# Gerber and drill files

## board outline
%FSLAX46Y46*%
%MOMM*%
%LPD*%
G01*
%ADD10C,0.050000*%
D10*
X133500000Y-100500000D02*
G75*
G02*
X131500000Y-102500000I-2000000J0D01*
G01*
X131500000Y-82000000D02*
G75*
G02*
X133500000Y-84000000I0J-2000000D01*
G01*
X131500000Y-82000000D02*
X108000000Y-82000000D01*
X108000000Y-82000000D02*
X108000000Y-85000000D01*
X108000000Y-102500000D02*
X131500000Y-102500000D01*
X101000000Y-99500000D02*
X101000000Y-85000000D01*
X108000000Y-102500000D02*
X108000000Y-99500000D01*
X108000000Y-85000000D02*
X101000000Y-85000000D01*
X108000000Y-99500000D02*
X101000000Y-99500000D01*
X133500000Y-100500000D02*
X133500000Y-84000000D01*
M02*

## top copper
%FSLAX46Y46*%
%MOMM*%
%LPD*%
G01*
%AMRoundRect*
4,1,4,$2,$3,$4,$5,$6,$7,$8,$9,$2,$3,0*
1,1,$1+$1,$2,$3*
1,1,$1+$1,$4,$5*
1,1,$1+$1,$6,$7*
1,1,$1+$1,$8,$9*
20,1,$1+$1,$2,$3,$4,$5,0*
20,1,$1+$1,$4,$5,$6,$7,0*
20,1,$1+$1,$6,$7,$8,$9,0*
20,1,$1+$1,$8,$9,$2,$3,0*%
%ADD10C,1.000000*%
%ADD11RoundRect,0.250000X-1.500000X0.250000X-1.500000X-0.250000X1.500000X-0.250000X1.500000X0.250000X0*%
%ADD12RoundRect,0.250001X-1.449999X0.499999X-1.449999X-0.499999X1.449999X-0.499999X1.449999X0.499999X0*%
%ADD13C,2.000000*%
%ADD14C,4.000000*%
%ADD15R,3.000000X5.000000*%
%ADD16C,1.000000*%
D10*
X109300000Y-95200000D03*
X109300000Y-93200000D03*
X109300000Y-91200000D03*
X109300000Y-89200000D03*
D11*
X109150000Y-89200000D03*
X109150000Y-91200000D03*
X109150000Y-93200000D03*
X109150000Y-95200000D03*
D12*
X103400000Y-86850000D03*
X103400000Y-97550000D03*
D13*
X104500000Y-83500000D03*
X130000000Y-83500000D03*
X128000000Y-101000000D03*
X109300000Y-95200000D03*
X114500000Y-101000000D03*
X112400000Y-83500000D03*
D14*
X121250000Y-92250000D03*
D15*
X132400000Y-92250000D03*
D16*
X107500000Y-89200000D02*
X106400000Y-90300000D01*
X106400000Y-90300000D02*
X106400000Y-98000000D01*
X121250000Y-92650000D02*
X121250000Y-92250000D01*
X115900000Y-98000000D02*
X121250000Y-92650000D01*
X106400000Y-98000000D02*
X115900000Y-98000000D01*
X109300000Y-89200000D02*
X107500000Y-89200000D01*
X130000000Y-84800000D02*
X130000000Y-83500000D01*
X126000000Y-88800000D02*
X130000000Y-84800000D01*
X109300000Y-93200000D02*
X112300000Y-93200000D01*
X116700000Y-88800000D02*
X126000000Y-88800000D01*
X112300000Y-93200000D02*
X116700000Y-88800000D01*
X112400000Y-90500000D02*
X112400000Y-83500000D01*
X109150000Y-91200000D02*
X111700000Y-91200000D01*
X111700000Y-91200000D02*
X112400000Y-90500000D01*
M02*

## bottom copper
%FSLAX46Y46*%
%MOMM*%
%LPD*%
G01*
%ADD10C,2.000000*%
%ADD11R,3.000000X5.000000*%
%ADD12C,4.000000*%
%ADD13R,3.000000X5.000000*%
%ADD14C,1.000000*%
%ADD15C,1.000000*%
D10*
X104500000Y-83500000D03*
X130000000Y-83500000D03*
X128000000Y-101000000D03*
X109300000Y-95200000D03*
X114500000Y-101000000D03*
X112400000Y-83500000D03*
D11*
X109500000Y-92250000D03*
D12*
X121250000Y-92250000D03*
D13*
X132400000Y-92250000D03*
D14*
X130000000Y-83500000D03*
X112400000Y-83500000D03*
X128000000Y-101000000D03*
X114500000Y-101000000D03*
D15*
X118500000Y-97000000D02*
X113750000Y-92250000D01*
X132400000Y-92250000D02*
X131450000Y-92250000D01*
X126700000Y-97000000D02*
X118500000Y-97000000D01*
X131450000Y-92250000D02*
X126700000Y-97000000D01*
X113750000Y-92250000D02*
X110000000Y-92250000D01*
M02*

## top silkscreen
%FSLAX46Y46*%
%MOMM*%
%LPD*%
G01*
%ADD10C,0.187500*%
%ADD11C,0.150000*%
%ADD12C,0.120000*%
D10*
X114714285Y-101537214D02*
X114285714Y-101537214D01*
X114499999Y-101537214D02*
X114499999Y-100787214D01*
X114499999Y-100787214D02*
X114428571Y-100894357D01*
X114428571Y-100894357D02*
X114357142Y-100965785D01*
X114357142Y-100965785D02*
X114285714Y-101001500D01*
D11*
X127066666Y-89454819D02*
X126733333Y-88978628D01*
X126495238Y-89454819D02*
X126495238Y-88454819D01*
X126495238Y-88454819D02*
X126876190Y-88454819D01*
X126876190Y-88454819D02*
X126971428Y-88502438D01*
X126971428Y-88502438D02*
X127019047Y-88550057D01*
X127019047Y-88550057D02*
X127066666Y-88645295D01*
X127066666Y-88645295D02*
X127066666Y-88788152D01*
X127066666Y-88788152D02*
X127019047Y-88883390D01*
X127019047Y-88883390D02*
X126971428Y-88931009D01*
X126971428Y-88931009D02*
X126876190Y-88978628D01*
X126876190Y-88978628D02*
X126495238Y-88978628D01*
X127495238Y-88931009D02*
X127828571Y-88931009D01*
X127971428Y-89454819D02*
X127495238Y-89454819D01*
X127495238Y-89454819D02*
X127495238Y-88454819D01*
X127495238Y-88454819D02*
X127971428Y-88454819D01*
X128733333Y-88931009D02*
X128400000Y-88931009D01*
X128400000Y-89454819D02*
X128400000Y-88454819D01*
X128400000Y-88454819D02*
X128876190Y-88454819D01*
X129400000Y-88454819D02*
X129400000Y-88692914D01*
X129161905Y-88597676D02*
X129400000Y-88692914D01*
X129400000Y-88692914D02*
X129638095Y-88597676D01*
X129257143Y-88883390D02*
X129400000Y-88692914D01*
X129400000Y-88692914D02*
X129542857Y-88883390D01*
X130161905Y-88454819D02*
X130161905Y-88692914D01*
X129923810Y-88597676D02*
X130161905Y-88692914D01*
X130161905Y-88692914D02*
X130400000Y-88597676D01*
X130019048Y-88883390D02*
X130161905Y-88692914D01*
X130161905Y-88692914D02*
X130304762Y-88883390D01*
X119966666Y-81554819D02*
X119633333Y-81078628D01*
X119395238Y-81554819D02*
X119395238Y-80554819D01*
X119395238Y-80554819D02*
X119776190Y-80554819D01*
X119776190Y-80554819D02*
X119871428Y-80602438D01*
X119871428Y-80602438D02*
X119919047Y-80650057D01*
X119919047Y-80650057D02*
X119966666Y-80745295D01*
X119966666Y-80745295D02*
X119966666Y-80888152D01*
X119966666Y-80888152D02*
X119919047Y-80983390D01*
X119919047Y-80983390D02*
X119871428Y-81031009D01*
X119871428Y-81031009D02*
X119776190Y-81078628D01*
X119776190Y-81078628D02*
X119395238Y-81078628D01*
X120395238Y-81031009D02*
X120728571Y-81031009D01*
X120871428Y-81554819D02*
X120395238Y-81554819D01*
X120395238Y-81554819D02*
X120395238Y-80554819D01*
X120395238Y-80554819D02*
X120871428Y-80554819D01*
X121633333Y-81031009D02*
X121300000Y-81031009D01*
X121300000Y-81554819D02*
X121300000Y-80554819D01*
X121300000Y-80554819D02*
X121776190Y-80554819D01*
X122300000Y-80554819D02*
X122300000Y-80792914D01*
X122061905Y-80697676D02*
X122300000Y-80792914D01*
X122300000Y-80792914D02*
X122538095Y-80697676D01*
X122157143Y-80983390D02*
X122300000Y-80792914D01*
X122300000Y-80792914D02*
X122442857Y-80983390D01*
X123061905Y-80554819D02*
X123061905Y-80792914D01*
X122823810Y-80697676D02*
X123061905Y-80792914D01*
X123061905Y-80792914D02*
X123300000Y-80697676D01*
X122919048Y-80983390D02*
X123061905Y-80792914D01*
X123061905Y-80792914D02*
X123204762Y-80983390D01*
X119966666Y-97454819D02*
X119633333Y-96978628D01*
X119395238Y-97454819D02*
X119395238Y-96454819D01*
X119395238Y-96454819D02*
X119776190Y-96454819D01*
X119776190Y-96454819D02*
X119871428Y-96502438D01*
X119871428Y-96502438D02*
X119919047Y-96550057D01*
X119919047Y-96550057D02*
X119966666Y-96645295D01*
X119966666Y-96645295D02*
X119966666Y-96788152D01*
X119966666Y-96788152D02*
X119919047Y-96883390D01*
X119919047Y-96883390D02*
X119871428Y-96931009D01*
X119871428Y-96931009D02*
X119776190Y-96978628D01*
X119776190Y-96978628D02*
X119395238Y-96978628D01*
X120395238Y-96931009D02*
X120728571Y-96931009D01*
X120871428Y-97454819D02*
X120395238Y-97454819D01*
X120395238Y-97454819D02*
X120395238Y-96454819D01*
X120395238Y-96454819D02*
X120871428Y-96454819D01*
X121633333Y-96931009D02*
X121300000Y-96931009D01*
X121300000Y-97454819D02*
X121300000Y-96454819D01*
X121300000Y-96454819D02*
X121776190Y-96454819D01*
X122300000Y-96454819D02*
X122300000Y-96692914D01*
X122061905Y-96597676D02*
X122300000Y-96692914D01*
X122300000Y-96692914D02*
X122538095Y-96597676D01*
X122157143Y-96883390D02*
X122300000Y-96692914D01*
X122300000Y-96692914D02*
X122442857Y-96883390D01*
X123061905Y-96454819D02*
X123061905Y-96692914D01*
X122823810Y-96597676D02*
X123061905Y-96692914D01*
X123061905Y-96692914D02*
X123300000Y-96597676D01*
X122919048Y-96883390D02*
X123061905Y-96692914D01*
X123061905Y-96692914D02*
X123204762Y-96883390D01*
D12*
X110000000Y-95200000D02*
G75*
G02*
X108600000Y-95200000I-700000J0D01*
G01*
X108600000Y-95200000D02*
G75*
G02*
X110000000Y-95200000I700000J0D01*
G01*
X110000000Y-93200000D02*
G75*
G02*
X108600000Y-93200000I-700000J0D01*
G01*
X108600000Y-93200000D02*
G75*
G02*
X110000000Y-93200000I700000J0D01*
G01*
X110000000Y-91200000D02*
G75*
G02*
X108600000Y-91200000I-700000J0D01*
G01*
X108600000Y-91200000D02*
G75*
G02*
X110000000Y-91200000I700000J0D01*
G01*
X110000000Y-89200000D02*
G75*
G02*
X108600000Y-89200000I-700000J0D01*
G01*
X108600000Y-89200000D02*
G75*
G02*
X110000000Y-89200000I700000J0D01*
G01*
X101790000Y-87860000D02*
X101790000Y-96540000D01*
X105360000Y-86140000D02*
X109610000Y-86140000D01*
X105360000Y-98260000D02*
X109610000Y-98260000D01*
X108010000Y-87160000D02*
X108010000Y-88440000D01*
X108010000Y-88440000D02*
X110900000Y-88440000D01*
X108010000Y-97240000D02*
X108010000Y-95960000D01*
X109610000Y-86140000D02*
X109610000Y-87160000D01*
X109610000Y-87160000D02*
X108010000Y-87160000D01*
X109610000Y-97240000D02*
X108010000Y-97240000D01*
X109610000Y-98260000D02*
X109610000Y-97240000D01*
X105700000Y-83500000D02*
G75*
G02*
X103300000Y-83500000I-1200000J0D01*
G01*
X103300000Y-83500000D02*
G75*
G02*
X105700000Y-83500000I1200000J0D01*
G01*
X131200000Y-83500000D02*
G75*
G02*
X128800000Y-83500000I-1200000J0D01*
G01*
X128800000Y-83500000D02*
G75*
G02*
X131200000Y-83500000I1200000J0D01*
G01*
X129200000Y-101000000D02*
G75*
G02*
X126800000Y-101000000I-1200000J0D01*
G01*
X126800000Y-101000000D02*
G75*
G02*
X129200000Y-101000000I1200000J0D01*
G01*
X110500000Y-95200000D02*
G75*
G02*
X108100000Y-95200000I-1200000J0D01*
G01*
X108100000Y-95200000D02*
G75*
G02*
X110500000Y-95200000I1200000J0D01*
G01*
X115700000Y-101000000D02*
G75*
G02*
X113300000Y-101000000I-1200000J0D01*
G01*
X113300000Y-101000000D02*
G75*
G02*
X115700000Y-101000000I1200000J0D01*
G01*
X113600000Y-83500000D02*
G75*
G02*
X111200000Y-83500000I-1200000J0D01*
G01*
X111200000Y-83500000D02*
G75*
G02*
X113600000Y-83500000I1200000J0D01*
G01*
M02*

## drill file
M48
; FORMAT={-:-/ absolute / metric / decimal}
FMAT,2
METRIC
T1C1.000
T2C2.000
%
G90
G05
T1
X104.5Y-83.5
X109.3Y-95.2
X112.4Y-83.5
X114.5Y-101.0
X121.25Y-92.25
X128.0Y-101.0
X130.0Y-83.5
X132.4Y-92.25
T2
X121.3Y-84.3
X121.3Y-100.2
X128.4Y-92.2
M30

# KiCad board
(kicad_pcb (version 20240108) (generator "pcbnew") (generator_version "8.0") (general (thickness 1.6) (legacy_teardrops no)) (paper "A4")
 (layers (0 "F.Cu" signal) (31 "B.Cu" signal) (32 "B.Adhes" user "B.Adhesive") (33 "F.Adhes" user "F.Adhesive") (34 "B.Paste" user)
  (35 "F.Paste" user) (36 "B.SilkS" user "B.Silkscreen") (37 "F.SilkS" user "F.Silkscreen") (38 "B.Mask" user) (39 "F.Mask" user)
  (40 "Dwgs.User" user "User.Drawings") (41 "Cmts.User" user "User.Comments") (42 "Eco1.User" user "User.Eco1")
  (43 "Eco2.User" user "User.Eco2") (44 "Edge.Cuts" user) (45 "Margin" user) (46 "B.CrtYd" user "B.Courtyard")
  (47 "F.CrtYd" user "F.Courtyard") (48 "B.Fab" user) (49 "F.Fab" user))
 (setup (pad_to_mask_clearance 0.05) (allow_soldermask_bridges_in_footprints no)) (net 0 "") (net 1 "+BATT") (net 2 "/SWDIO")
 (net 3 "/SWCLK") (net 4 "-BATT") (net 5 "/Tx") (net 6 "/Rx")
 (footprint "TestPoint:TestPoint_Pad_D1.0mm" (layer "F.Cu") (at 109.3 95.2)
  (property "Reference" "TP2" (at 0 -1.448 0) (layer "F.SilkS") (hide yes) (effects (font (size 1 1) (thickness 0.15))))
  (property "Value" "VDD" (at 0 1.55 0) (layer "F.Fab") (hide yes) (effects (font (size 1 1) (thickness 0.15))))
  (fp_circle (center 0 0) (end 0 0.7) (stroke (width 0.12) (type solid)) (fill none) (layer "F.SilkS"))
  (pad "1" smd circle (at 0 0) (size 1 1) (layers "F.Cu" "F.Mask") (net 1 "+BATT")))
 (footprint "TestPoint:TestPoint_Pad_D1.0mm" (layer "F.Cu") (at 109.3 93.2)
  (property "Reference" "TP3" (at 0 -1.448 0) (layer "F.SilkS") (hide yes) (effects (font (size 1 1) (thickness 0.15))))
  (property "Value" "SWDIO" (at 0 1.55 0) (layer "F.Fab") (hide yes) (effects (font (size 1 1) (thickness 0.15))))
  (fp_circle (center 0 0) (end 0 0.7) (stroke (width 0.12) (type solid)) (fill none) (layer "F.SilkS"))
  (pad "1" smd circle (at 0 0) (size 1 1) (layers "F.Cu" "F.Mask") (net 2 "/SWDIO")))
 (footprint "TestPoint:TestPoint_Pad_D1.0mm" (layer "F.Cu") (at 109.3 91.2)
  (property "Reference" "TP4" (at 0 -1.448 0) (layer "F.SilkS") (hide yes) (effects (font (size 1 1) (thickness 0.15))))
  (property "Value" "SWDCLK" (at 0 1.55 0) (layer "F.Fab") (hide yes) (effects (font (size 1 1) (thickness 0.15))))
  (fp_circle (center 0 0) (end 0 0.7) (stroke (width 0.12) (type solid)) (fill none) (layer "F.SilkS"))
  (pad "1" smd circle (at 0 0) (size 1 1) (layers "F.Cu" "F.Mask") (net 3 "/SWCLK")))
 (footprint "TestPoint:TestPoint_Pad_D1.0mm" (layer "F.Cu") (at 109.3 89.2)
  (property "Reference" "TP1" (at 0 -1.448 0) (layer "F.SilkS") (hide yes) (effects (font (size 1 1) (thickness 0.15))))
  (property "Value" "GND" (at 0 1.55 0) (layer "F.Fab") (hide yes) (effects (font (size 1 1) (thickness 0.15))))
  (fp_circle (center 0 0) (end 0 0.7) (stroke (width 0.12) (type solid)) (fill none) (layer "F.SilkS"))
  (pad "1" smd circle (at 0 0) (size 1 1) (layers "F.Cu" "F.Mask") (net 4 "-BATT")))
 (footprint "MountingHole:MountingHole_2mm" (layer "F.Cu") (at 128.4 92.2)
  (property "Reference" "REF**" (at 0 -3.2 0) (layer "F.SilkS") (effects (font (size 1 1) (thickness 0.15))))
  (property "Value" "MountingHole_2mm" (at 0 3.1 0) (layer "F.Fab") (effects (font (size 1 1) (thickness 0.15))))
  (pad "" np_thru_hole circle (at 0 0) (size 2 2) (drill 2) (layers "*.Cu" "*.Mask")))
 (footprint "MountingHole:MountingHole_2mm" (layer "F.Cu") (at 121.3 84.3)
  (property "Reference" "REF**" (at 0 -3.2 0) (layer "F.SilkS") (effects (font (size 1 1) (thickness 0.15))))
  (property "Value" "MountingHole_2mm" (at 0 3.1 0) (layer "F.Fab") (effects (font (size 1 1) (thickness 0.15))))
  (pad "" np_thru_hole circle (at 0 0) (size 2 2) (drill 2) (layers "*.Cu" "*.Mask")))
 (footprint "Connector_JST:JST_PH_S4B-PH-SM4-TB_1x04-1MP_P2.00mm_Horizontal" (layer "F.Cu") (at 106.3 92.2 -90)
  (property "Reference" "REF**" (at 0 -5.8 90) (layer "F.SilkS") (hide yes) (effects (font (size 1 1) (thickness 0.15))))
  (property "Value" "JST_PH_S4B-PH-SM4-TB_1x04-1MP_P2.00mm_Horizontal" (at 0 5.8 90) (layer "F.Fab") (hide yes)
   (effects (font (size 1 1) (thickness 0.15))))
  (fp_line (start -4.34 4.51) (end 4.34 4.51) (stroke (width 0.12) (type solid)) (layer "F.SilkS"))
  (fp_line (start -6.06 0.94) (end -6.06 -3.31) (stroke (width 0.12) (type solid)) (layer "F.SilkS"))
  (fp_line (start 6.06 0.94) (end 6.06 -3.31) (stroke (width 0.12) (type solid)) (layer "F.SilkS"))
  (fp_line (start -5.04 -1.71) (end -3.76 -1.71) (stroke (width 0.12) (type solid)) (layer "F.SilkS"))
  (fp_line (start -3.76 -1.71) (end -3.76 -4.6) (stroke (width 0.12) (type solid)) (layer "F.SilkS"))
  (fp_line (start 5.04 -1.71) (end 3.76 -1.71) (stroke (width 0.12) (type solid)) (layer "F.SilkS"))
  (fp_line (start -6.06 -3.31) (end -5.04 -3.31) (stroke (width 0.12) (type solid)) (layer "F.SilkS"))
  (fp_line (start -5.04 -3.31) (end -5.04 -1.71) (stroke (width 0.12) (type solid)) (layer "F.SilkS"))
  (fp_line (start 5.04 -3.31) (end 5.04 -1.71) (stroke (width 0.12) (type solid)) (layer "F.SilkS"))
  (fp_line (start 6.06 -3.31) (end 5.04 -3.31) (stroke (width 0.12) (type solid)) (layer "F.SilkS"))
  (pad "1" smd roundrect (at -3 -2.85 270) (size 1 3.5) (layers "F.Cu" "F.Paste" "F.Mask") (roundrect_rratio 0.25) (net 4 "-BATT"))
  (pad "2" smd roundrect (at -1 -2.85 270) (size 1 3.5) (layers "F.Cu" "F.Paste" "F.Mask") (roundrect_rratio 0.25) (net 3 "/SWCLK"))
  (pad "3" smd roundrect (at 1 -2.85 270) (size 1 3.5) (layers "F.Cu" "F.Paste" "F.Mask") (roundrect_rratio 0.25) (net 2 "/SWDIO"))
  (pad "4" smd roundrect (at 3 -2.85 270) (size 1 3.5) (layers "F.Cu" "F.Paste" "F.Mask") (roundrect_rratio 0.25) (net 1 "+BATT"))
  (pad "MP" smd roundrect (at -5.35 2.9 270) (size 1.5 3.4) (layers "F.Cu" "F.Paste" "F.Mask") (roundrect_rratio 0.166667))
  (pad "MP" smd roundrect (at 5.35 2.9 270) (size 1.5 3.4) (layers "F.Cu" "F.Paste" "F.Mask") (roundrect_rratio 0.166667)))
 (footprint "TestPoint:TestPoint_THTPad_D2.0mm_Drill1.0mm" (layer "F.Cu") (at 104.5 83.5)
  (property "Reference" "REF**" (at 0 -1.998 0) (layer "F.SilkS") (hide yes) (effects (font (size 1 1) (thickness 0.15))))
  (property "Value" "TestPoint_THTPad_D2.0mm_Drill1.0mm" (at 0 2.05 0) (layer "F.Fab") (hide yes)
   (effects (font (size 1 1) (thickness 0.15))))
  (fp_circle (center 0 0) (end 0 1.2) (stroke (width 0.12) (type solid)) (fill none) (layer "F.SilkS"))
  (pad "1" thru_hole circle (at 0 0) (size 2 2) (drill 1) (layers "*.Cu" "*.Mask") (remove_unused_layers no)))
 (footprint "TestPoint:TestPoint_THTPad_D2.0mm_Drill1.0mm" (layer "F.Cu") (at 130 83.5)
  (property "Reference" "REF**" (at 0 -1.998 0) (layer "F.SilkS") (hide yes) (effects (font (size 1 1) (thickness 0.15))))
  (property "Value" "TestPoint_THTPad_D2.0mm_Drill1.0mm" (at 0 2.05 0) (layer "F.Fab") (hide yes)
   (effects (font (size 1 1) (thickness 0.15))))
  (fp_circle (center 0 0) (end 0 1.2) (stroke (width 0.12) (type solid)) (fill none) (layer "F.SilkS"))
  (pad "1" thru_hole circle (at 0 0) (size 2 2) (drill 1) (layers "*.Cu" "*.Mask") (remove_unused_layers no) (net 2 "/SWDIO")))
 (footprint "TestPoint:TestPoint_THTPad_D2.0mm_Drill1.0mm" (layer "F.Cu") (at 128 101)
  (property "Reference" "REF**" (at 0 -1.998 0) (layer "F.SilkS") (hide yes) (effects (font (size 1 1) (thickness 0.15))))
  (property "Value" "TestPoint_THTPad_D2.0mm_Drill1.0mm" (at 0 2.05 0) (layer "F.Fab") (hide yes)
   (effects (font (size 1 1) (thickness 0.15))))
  (fp_circle (center 0 0) (end 0 1.2) (stroke (width 0.12) (type solid)) (fill none) (layer "F.SilkS"))
  (pad "1" thru_hole circle (at 0 0) (size 2 2) (drill 1) (layers "*.Cu" "*.Mask") (remove_unused_layers no) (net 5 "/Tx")))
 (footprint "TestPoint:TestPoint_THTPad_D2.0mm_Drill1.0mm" (layer "F.Cu") (at 109.3 95.2)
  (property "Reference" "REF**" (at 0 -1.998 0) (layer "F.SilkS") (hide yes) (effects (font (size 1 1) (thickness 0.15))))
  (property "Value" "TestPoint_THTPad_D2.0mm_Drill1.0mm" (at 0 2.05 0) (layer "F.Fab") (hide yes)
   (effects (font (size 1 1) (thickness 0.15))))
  (fp_circle (center 0 0) (end 0 1.2) (stroke (width 0.12) (type solid)) (fill none) (layer "F.SilkS"))
  (pad "1" thru_hole circle (at 0 0) (size 2 2) (drill 1) (layers "*.Cu" "*.Mask") (remove_unused_layers no) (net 1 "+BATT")))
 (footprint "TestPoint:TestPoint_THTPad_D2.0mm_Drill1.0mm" (layer "F.Cu") (at 114.5 101)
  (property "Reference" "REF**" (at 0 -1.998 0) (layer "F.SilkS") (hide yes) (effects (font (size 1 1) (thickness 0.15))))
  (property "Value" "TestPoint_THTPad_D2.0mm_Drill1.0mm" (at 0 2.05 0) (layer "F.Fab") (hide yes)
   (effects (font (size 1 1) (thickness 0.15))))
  (fp_circle (center 0 0) (end 0 1.2) (stroke (width 0.12) (type solid)) (fill none) (layer "F.SilkS"))
  (pad "1" thru_hole circle (at 0 0) (size 2 2) (drill 1) (layers "*.Cu" "*.Mask") (remove_unused_layers no) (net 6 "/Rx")))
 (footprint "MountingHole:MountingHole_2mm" (layer "F.Cu") (at 121.3 100.2)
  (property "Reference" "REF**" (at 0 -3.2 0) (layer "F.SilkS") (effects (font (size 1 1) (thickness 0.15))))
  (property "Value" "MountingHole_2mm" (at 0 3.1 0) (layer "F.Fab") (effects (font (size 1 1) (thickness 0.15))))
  (pad "" np_thru_hole circle (at 0 0) (size 2 2) (drill 2) (layers "*.Cu" "*.Mask")))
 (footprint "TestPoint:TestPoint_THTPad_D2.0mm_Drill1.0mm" (layer "F.Cu") (at 112.4 83.5)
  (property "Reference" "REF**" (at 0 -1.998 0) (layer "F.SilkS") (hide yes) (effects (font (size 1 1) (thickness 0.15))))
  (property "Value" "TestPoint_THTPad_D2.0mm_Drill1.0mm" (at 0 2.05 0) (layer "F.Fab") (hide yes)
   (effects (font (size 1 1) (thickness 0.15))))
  (fp_circle (center 0 0) (end 0 1.2) (stroke (width 0.12) (type solid)) (fill none) (layer "F.SilkS"))
  (pad "1" thru_hole circle (at 0 0) (size 2 2) (drill 1) (layers "*.Cu" "*.Mask") (remove_unused_layers no) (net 3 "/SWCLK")))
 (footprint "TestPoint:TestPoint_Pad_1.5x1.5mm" (layer "B.Cu") (at 110 92.25)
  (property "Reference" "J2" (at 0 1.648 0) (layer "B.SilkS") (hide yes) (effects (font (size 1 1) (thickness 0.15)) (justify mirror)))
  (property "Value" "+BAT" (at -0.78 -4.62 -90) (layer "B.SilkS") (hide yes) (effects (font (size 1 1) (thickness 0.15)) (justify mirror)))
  (pad "1" smd rect (at 0 0) (size 3 5) (drill (offset -0.5 0)) (layers "B.Cu" "B.Mask") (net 1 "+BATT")))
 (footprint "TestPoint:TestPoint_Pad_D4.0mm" (layer "B.Cu") (at 121.25 92.25)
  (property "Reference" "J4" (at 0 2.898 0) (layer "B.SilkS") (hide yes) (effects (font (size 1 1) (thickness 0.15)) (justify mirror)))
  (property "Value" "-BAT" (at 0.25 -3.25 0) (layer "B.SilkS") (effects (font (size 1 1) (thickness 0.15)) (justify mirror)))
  (pad "1" thru_hole circle (at 0 0) (size 4 4) (drill 1) (layers "*.Cu" "*.Mask") (remove_unused_layers no) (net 4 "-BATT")))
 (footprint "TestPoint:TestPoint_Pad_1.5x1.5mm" (layer "B.Cu") (at 132.4 92.25)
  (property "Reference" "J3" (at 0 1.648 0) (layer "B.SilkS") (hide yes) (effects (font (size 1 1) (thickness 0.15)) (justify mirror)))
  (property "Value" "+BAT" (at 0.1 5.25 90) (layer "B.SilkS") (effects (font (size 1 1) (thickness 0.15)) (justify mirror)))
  (pad "1" thru_hole rect (at 0 0) (size 3 5) (drill 1) (layers "*.Cu" "*.Mask") (remove_unused_layers no) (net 1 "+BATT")))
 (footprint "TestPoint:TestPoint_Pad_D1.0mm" (layer "B.Cu") (at 130 83.5)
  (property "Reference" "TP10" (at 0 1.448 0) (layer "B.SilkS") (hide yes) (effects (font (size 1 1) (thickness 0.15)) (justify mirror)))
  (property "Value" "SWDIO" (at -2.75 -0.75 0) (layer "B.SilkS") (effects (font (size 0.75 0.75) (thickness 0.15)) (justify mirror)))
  (pad "1" smd circle (at 0 0) (size 1 1) (layers "B.Cu" "B.Mask") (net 2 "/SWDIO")))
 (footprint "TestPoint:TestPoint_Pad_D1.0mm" (layer "B.Cu") (at 112.4 83.5)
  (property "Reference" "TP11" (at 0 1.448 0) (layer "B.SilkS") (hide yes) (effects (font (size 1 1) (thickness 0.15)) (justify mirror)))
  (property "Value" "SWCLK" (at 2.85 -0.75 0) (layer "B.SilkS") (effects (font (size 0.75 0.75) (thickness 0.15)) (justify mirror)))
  (pad "1" smd circle (at 0 0) (size 1 1) (layers "B.Cu" "B.Mask") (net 3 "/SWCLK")))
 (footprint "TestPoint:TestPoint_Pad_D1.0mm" (layer "B.Cu") (at 128 101 180)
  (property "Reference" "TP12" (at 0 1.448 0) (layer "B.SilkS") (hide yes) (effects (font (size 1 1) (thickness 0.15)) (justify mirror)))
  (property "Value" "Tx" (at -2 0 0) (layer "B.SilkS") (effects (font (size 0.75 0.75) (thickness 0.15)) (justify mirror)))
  (pad "1" smd circle (at 0 0 180) (size 1 1) (layers "B.Cu" "B.Mask") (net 5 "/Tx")))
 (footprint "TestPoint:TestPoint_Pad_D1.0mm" (layer "B.Cu") (at 114.5 101 180)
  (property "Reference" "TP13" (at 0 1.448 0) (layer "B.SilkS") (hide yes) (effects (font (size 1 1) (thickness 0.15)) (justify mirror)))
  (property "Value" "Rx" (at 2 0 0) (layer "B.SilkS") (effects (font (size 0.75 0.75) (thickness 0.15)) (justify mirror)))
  (pad "1" smd circle (at 0 0 180) (size 1 1) (layers "B.Cu" "B.Mask") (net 6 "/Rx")))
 (gr_arc (start 133.5 100.5) (mid 132.914214 101.914214) (end 131.5 102.5) (stroke (width 0.05) (type solid)) (layer "Edge.Cuts"))
 (gr_arc (start 131.5 82) (mid 132.914214 82.585786) (end 133.5 84) (stroke (width 0.05) (type solid)) (layer "Edge.Cuts"))
 (gr_line (start 131.5 82) (end 108 82) (stroke (width 0.05) (type solid)) (layer "Edge.Cuts"))
 (gr_line (start 108 82) (end 108 85) (stroke (width 0.05) (type default)) (layer "Edge.Cuts"))
 (gr_line (start 108 102.5) (end 131.5 102.5) (stroke (width 0.05) (type solid)) (layer "Edge.Cuts"))
 (gr_line (start 101 99.5) (end 101 85) (stroke (width 0.05) (type default)) (layer "Edge.Cuts"))
 (gr_line (start 108 102.5) (end 108 99.5) (stroke (width 0.05) (type default)) (layer "Edge.Cuts"))
 (gr_line (start 108 85) (end 101 85) (stroke (width 0.05) (type default)) (layer "Edge.Cuts"))
 (gr_line (start 108 99.5) (end 101 99.5) (stroke (width 0.05) (type default)) (layer "Edge.Cuts"))
 (gr_line (start 133.5 100.5) (end 133.5 84) (stroke (width 0.05) (type solid)) (layer "Edge.Cuts"))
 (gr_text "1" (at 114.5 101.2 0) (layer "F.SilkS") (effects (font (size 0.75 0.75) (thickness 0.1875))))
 (segment (start 118.5 97) (end 113.75 92.25) (width 1) (layer "B.Cu") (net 1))
 (segment (start 132.4 92.25) (end 131.45 92.25) (width 1) (layer "B.Cu") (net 1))
 (segment (start 126.7 97) (end 118.5 97) (width 1) (layer "B.Cu") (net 1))
 (segment (start 131.45 92.25) (end 126.7 97) (width 1) (layer "B.Cu") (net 1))
 (segment (start 113.75 92.25) (end 110 92.25) (width 1) (layer "B.Cu") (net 1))
 (segment (start 107.5 89.2) (end 106.4 90.3) (width 1) (layer "F.Cu") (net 4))
 (segment (start 106.4 90.3) (end 106.4 98) (width 1) (layer "F.Cu") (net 4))
 (segment (start 121.25 92.65) (end 121.25 92.25) (width 1) (layer "F.Cu") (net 4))
 (segment (start 115.9 98) (end 121.25 92.65) (width 1) (layer "F.Cu") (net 4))
 (segment (start 106.4 98) (end 115.9 98) (width 1) (layer "F.Cu") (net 4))
 (segment (start 109.3 89.2) (end 107.5 89.2) (width 1) (layer "F.Cu") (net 4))
 (segment (start 130 84.8) (end 130 83.5) (width 1) (layer "F.Cu") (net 2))
 (segment (start 126 88.8) (end 130 84.8) (width 1) (layer "F.Cu") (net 2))
 (segment (start 109.3 93.2) (end 112.3 93.2) (width 1) (layer "F.Cu") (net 2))
 (segment (start 116.7 88.8) (end 126 88.8) (width 1) (layer "F.Cu") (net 2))
 (segment (start 112.3 93.2) (end 116.7 88.8) (width 1) (layer "F.Cu") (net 2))
 (segment (start 112.4 90.5) (end 112.4 83.5) (width 1) (layer "F.Cu") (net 3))
 (segment (start 109.15 91.2) (end 111.7 91.2) (width 1) (layer "F.Cu") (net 3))
 (segment (start 111.7 91.2) (end 112.4 90.5) (width 1) (layer "F.Cu") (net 3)))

